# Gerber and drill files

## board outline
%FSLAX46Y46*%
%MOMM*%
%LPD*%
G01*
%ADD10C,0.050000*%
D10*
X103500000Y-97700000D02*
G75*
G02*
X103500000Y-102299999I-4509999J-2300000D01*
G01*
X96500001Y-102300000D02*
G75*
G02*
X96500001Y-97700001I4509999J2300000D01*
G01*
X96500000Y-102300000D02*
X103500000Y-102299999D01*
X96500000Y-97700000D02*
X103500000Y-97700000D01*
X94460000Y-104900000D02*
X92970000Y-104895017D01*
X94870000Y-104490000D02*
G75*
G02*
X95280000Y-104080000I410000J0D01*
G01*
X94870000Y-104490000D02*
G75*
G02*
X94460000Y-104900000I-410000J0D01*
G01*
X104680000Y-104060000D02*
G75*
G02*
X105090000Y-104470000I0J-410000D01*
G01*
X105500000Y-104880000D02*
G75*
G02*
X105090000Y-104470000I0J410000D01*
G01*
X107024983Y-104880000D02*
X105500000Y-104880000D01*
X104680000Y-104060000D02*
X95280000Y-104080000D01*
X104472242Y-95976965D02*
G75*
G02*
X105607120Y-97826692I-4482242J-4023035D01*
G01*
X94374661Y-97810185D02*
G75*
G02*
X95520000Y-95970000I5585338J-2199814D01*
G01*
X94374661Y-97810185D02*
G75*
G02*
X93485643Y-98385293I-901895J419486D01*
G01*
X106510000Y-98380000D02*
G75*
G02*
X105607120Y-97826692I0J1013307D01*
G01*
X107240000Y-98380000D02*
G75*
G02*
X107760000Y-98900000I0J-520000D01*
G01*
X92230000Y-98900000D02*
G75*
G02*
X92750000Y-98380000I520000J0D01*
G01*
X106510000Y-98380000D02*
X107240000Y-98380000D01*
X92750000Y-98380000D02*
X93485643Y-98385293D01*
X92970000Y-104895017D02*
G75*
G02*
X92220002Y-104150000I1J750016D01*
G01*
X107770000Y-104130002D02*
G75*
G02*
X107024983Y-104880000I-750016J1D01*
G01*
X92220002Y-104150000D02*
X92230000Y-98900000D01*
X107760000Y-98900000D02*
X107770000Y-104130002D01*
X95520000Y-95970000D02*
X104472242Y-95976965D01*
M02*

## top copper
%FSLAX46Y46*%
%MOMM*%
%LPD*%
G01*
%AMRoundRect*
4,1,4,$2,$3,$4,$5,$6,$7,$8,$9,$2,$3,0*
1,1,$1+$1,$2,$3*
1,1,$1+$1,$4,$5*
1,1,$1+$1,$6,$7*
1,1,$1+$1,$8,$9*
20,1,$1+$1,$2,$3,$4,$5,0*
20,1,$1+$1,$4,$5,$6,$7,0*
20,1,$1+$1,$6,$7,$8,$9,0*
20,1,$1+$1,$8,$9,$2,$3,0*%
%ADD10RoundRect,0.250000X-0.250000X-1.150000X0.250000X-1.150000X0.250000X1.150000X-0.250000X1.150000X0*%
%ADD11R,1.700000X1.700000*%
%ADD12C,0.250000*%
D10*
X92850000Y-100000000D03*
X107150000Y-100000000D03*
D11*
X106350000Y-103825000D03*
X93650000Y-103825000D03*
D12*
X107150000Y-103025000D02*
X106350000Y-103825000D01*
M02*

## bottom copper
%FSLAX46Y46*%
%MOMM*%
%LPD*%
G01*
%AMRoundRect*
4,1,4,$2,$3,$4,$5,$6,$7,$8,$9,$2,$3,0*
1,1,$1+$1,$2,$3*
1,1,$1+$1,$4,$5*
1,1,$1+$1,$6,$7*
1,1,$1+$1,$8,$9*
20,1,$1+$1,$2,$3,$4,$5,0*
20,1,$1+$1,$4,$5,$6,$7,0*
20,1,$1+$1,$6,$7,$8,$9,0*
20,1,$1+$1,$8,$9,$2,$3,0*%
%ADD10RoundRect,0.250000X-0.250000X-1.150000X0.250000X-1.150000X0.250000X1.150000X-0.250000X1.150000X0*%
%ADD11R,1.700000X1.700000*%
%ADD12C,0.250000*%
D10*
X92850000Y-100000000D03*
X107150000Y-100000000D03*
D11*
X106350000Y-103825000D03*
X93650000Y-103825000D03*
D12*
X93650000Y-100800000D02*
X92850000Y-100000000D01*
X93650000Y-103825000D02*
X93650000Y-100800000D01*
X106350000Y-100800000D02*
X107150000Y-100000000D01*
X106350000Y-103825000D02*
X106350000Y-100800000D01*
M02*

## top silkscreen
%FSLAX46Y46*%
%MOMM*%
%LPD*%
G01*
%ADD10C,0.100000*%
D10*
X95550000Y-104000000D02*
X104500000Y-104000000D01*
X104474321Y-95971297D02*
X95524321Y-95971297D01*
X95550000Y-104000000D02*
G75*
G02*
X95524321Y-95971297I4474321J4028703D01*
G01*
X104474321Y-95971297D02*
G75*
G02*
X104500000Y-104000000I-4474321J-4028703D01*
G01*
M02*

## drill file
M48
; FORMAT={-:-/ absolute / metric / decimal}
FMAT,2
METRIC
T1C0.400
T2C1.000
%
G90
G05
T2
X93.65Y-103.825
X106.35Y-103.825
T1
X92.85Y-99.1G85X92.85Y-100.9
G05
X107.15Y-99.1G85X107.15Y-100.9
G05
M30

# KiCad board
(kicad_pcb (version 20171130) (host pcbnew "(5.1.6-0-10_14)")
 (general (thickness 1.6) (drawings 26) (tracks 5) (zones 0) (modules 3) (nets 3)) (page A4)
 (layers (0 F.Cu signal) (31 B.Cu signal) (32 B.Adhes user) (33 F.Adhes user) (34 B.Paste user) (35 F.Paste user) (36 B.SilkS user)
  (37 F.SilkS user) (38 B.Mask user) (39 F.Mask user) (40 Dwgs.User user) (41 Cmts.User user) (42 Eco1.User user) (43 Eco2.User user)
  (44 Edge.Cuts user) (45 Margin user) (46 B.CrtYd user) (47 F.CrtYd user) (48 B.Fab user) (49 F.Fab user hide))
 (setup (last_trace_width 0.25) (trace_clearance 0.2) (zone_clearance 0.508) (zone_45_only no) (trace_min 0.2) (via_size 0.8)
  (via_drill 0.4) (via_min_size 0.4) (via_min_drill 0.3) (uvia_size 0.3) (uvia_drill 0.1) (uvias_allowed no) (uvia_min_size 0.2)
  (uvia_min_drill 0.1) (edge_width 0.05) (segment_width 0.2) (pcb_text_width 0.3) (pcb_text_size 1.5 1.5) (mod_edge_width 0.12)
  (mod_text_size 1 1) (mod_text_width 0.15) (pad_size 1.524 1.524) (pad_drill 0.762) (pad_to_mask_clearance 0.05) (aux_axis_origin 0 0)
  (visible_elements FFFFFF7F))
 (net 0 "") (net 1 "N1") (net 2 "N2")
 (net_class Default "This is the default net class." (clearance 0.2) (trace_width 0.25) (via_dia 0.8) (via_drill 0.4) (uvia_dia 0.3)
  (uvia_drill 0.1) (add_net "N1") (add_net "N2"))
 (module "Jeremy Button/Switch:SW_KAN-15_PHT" (layer F.Cu) (at 100 100)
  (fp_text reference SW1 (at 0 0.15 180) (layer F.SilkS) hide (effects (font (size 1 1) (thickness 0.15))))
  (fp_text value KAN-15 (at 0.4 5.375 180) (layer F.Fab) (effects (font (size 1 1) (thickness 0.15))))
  (fp_line (start -4.45 4) (end 4.5 4) (layer F.SilkS) (width 0.1))
  (fp_line (start 4.474321 -4.028703) (end -4.475679 -4.028703) (layer F.SilkS) (width 0.1))
  (fp_arc (start 0.024321 -0.028703) (end -4.475679 -4.028703) (angle -83.63358372) (layer F.SilkS) (width 0.1))
  (fp_arc (start 0 0) (end 4.5 4) (angle -83.63358372) (layer F.SilkS) (width 0.1))
  (pad 1 thru_hole roundrect (at -7.15 0) (size 1 2.8) (drill oval 0.4 2.2) (layers *.Cu *.Mask) (roundrect_rratio 0.25) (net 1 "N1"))
  (pad 2 thru_hole roundrect (at 7.15 0) (size 1 2.8) (drill oval 0.4 2.2) (layers *.Cu *.Mask) (roundrect_rratio 0.25) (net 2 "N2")))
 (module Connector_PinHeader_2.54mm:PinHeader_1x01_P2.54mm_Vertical (layer F.Cu) (at 106.35 103.825 180)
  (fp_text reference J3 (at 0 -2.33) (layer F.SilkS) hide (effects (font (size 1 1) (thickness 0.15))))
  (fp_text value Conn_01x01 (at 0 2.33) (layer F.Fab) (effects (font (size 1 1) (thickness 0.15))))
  (pad 1 thru_hole rect (at 0 0 180) (size 1.7 1.7) (drill 1) (layers *.Cu *.Mask) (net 2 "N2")))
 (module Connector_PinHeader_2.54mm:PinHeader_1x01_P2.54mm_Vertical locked (layer F.Cu) (at 93.65 103.825 90)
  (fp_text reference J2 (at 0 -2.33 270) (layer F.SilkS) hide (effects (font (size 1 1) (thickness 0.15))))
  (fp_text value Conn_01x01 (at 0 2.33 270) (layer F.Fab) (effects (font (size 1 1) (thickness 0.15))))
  (pad 1 thru_hole rect (at 0 0 90) (size 1.7 1.7) (drill 1) (layers *.Cu *.Mask) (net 1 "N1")))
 (gr_arc (start 98.990001 100) (end 103.5 102.299999) (angle -54.04114679) (layer Edge.Cuts) (width 0.05))
 (gr_arc (start 101.01 100) (end 96.500001 97.700001) (angle -54.04114679) (layer Edge.Cuts) (width 0.05))
 (gr_line (start 96.5 102.3) (end 103.5 102.299999) (layer Edge.Cuts) (width 0.05))
 (gr_line (start 96.5 97.7) (end 103.5 97.7) (layer Edge.Cuts) (width 0.05))
 (gr_line (start 94.46 104.9) (end 92.97 104.895017) (layer Edge.Cuts) (width 0.05))
 (gr_arc (start 95.28 104.49) (end 95.28 104.08) (angle -90) (layer Edge.Cuts) (width 0.05))
 (gr_arc (start 94.46 104.49) (end 94.46 104.9) (angle -90) (layer Edge.Cuts) (width 0.05))
 (gr_arc (start 104.68 104.47) (end 105.09 104.47) (angle -90) (layer Edge.Cuts) (width 0.05))
 (gr_arc (start 105.5 104.47) (end 105.09 104.47) (angle -90) (layer Edge.Cuts) (width 0.05))
 (gr_line (start 107.024983 104.88) (end 105.5 104.88) (layer Edge.Cuts) (width 0.05))
 (gr_line (start 104.68 104.06) (end 95.28 104.08) (layer Edge.Cuts) (width 0.05))
 (gr_arc (start 99.99 100) (end 105.60712 97.826692) (angle -20.75770678) (layer Edge.Cuts) (width 0.05))
 (gr_arc (start 99.959999 100.009999) (end 95.52 95.97) (angle -20.80211291) (layer Edge.Cuts) (width 0.05))
 (gr_arc (start 93.472766 97.390699) (end 93.485643 98.385293) (angle -64.31433064) (layer Edge.Cuts) (width 0.05))
 (gr_arc (start 106.51 97.366693) (end 105.60712 97.826692) (angle -63.00205791) (layer Edge.Cuts) (width 0.05))
 (gr_arc (start 107.24 98.9) (end 107.76 98.9) (angle -90) (layer Edge.Cuts) (width 0.05))
 (gr_arc (start 92.75 98.9) (end 92.75 98.38) (angle -90) (layer Edge.Cuts) (width 0.05))
 (gr_line (start 106.51 98.38) (end 107.24 98.38) (layer Edge.Cuts) (width 0.05))
 (gr_line (start 92.75 98.38) (end 93.485643 98.385293) (layer Edge.Cuts) (width 0.05))
 (gr_arc (start 92.970001 104.145001) (end 92.220002 104.15) (angle -89.6180338) (layer Edge.Cuts) (width 0.05))
 (gr_arc (start 107.019984 104.130001) (end 107.024983 104.88) (angle -89.6180338) (layer Edge.Cuts) (width 0.05))
 (gr_line (start 92.220002 104.15) (end 92.23 98.9) (layer Edge.Cuts) (width 0.05))
 (gr_line (start 107.76 98.9) (end 107.77 104.130002) (layer Edge.Cuts) (width 0.05))
 (gr_line (start 95.52 95.97) (end 104.472242 95.976965) (layer Edge.Cuts) (width 0.05))
 (segment (start 93.65 100.8) (end 92.85 100) (width 0.25) (layer B.Cu) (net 1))
 (segment (start 93.65 103.825) (end 93.65 100.8) (width 0.25) (layer B.Cu) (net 1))
 (segment (start 107.15 103.025) (end 106.35 103.825) (width 0.25) (layer F.Cu) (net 2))
 (segment (start 106.35 100.8) (end 107.15 100) (width 0.25) (layer B.Cu) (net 2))
 (segment (start 106.35 103.825) (end 106.35 100.8) (width 0.25) (layer B.Cu) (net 2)))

